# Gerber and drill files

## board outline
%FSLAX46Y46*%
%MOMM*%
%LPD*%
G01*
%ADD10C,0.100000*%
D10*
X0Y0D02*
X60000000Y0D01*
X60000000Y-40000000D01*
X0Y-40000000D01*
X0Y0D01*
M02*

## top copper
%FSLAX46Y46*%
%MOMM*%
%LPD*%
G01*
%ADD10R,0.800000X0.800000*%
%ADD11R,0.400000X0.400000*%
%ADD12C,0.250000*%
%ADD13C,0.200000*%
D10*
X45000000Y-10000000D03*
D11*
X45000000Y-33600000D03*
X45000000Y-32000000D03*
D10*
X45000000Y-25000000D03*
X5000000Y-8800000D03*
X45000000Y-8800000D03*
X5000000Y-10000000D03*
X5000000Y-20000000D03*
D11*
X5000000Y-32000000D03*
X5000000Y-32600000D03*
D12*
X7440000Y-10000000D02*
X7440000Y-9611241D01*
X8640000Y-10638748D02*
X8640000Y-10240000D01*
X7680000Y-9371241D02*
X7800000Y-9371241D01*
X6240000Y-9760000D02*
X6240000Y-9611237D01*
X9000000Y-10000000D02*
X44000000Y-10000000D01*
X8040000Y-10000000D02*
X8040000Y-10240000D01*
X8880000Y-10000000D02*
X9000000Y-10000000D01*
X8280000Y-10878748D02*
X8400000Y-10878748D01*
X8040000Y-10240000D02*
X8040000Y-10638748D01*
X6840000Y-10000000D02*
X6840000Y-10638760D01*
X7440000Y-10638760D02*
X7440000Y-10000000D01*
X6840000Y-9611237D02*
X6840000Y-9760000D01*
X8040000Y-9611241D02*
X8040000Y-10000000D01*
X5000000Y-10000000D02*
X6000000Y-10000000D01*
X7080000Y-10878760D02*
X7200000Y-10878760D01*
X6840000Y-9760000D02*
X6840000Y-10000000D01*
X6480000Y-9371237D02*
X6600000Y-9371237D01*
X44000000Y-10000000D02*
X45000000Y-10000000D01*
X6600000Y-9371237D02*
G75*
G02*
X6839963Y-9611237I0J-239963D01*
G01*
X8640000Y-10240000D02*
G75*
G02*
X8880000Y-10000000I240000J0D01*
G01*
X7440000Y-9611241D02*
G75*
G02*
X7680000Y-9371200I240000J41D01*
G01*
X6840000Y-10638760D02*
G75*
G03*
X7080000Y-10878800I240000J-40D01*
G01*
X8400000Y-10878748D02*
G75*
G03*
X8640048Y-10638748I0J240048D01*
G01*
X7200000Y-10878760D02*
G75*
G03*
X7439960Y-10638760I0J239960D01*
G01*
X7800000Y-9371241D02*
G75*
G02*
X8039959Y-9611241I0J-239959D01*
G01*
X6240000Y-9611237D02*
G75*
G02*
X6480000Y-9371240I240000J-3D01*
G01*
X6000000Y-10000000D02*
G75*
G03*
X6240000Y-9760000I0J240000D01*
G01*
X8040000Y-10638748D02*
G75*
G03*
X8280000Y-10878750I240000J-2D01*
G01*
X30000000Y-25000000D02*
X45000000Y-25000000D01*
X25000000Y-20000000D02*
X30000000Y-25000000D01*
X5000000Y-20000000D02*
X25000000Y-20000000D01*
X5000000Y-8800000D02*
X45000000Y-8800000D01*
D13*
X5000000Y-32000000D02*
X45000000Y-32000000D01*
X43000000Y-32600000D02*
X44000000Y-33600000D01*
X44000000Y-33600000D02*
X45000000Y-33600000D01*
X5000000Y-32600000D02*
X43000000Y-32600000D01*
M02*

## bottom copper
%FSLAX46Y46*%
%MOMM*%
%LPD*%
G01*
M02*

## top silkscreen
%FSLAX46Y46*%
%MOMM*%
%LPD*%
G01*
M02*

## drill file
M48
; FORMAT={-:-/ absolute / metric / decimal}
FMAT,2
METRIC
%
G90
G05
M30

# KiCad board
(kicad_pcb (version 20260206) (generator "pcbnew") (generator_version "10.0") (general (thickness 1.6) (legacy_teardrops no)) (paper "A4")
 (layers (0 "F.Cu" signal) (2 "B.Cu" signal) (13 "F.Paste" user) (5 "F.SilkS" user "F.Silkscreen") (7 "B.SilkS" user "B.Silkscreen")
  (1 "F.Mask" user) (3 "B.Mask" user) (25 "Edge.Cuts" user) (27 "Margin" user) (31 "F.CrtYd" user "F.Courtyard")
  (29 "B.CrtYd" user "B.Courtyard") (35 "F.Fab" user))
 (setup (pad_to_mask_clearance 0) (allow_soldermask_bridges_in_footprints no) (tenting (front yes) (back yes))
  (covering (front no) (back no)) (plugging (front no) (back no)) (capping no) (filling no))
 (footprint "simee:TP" (layer "F.Cu") (at 45 10)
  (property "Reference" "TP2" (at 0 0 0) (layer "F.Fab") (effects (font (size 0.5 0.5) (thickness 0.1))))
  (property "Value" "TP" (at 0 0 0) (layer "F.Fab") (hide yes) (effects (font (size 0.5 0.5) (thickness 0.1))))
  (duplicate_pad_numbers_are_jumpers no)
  (pad "1" smd rect (at 0 0) (size 0.8 0.8) (layers "F.Cu" "F.Mask") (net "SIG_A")))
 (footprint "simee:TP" (layer "F.Cu") (at 45 33.6)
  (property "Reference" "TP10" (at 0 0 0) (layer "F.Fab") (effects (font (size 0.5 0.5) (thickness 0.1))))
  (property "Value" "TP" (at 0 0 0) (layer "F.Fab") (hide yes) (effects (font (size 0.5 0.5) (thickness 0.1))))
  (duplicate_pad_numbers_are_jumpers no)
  (pad "1" smd rect (at 0 0) (size 0.4 0.4) (layers "F.Cu" "F.Mask") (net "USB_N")))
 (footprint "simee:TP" (layer "F.Cu") (at 45 32)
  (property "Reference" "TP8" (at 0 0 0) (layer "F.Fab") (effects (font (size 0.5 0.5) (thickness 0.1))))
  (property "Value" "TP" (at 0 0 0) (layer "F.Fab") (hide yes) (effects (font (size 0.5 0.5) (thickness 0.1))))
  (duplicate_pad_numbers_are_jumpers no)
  (pad "1" smd rect (at 0 0) (size 0.4 0.4) (layers "F.Cu" "F.Mask") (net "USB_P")))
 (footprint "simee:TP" (layer "F.Cu") (at 45 25)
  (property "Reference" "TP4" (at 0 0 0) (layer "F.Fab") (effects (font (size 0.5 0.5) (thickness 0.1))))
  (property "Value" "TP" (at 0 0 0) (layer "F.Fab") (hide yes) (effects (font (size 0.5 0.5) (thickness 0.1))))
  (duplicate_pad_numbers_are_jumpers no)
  (pad "1" smd rect (at 0 0) (size 0.8 0.8) (layers "F.Cu" "F.Mask") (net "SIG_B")))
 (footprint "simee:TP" (layer "F.Cu") (at 5 8.8)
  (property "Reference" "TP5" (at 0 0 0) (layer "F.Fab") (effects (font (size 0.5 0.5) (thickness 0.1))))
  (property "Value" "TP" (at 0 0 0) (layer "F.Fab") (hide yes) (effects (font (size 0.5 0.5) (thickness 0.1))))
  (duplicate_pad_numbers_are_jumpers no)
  (pad "1" smd rect (at 0 0) (size 0.8 0.8) (layers "F.Cu" "F.Mask") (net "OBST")))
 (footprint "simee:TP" (layer "F.Cu") (at 45 8.8)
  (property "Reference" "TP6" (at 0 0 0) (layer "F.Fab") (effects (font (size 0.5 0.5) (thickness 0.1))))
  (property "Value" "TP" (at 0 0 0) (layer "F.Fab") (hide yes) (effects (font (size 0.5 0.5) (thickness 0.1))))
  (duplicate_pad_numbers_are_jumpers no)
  (pad "1" smd rect (at 0 0) (size 0.8 0.8) (layers "F.Cu" "F.Mask") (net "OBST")))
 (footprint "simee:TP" (layer "F.Cu") (at 5 10)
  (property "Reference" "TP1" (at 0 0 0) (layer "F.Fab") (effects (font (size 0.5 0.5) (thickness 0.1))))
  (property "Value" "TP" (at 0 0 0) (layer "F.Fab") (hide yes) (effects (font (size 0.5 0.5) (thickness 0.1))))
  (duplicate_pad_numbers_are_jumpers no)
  (pad "1" smd rect (at 0 0) (size 0.8 0.8) (layers "F.Cu" "F.Mask") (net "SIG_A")))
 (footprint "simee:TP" (layer "F.Cu") (at 5 20)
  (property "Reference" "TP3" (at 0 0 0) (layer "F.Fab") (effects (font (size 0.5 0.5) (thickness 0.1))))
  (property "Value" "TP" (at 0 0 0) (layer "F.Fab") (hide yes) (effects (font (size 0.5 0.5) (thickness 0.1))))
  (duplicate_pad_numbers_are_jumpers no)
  (pad "1" smd rect (at 0 0) (size 0.8 0.8) (layers "F.Cu" "F.Mask") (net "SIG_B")))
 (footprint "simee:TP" (layer "F.Cu") (at 5 32)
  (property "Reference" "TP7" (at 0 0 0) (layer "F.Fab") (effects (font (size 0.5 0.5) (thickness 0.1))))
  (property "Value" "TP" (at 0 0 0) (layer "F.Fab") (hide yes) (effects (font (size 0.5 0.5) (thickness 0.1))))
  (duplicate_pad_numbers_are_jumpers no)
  (pad "1" smd rect (at 0 0) (size 0.4 0.4) (layers "F.Cu" "F.Mask") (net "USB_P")))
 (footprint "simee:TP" (layer "F.Cu") (at 5 32.6)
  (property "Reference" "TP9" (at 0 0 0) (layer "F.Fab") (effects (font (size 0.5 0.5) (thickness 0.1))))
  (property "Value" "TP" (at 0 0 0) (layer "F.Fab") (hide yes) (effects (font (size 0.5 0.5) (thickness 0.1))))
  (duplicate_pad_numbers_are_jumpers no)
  (pad "1" smd rect (at 0 0) (size 0.4 0.4) (layers "F.Cu" "F.Mask") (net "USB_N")))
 (gr_rect (start 0 0) (end 60 40) (stroke (width 0.1) (type default)) (fill no) (layer "Edge.Cuts"))
 (segment (start 7.44 10) (end 7.44 9.611241) (width 0.25) (layer "F.Cu") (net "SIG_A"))
 (segment (start 8.64 10.638748) (end 8.64 10.24) (width 0.25) (layer "F.Cu") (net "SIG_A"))
 (segment (start 7.68 9.371241) (end 7.8 9.371241) (width 0.25) (layer "F.Cu") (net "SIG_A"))
 (segment (start 6.24 9.76) (end 6.24 9.611237) (width 0.25) (layer "F.Cu") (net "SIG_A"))
 (segment (start 9 10) (end 44 10) (width 0.25) (layer "F.Cu") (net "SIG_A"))
 (segment (start 8.04 10) (end 8.04 10.24) (width 0.25) (layer "F.Cu") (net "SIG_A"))
 (segment (start 8.88 10) (end 9 10) (width 0.25) (layer "F.Cu") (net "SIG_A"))
 (segment (start 8.28 10.878748) (end 8.4 10.878748) (width 0.25) (layer "F.Cu") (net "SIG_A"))
 (segment (start 8.04 10.24) (end 8.04 10.638748) (width 0.25) (layer "F.Cu") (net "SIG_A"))
 (segment (start 6.84 10) (end 6.84 10.63876) (width 0.25) (layer "F.Cu") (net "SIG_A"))
 (segment (start 7.44 10.63876) (end 7.44 10) (width 0.25) (layer "F.Cu") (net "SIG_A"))
 (segment (start 6.84 9.611237) (end 6.84 9.76) (width 0.25) (layer "F.Cu") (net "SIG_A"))
 (segment (start 8.04 9.611241) (end 8.04 10) (width 0.25) (layer "F.Cu") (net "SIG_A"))
 (segment (start 5 10) (end 6 10) (width 0.25) (layer "F.Cu") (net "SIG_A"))
 (segment (start 7.08 10.87876) (end 7.2 10.87876) (width 0.25) (layer "F.Cu") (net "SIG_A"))
 (segment (start 6.84 9.76) (end 6.84 10) (width 0.25) (layer "F.Cu") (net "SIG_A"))
 (segment (start 6.48 9.371237) (end 6.6 9.371237) (width 0.25) (layer "F.Cu") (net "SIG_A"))
 (segment (start 44 10) (end 45 10) (width 0.25) (layer "F.Cu") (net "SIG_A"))
 (arc (start 6.6 9.371237) (mid 6.769706 9.441531) (end 6.84 9.611237) (width 0.25) (layer "F.Cu") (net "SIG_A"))
 (arc (start 8.64 10.24) (mid 8.710294 10.070294) (end 8.88 10) (width 0.25) (layer "F.Cu") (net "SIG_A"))
 (arc (start 7.44 9.611241) (mid 7.510294 9.441535) (end 7.68 9.371241) (width 0.25) (layer "F.Cu") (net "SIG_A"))
 (arc (start 6.84 10.63876) (mid 6.910294 10.808466) (end 7.08 10.87876) (width 0.25) (layer "F.Cu") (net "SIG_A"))
 (arc (start 8.4 10.878748) (mid 8.569706 10.808454) (end 8.64 10.638748) (width 0.25) (layer "F.Cu") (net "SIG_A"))
 (arc (start 7.2 10.87876) (mid 7.369706 10.808466) (end 7.44 10.63876) (width 0.25) (layer "F.Cu") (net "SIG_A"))
 (arc (start 7.8 9.371241) (mid 7.969706 9.441535) (end 8.04 9.611241) (width 0.25) (layer "F.Cu") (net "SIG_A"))
 (arc (start 6.24 9.611237) (mid 6.310294 9.441531) (end 6.48 9.371237) (width 0.25) (layer "F.Cu") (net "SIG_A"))
 (arc (start 6 10) (mid 6.169706 9.929706) (end 6.24 9.76) (width 0.25) (layer "F.Cu") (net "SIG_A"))
 (arc (start 8.04 10.638748) (mid 8.110294 10.808454) (end 8.28 10.878748) (width 0.25) (layer "F.Cu") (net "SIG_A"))
 (segment (start 30 25) (end 45 25) (width 0.25) (layer "F.Cu") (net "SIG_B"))
 (segment (start 25 20) (end 30 25) (width 0.25) (layer "F.Cu") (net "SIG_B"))
 (segment (start 5 20) (end 25 20) (width 0.25) (layer "F.Cu") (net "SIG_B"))
 (segment (start 5 8.8) (end 45 8.8) (width 0.25) (layer "F.Cu") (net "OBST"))
 (segment (start 5 32) (end 45 32) (width 0.2) (layer "F.Cu") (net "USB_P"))
 (segment (start 43 32.6) (end 44 33.6) (width 0.2) (layer "F.Cu") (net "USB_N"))
 (segment (start 44 33.6) (end 45 33.6) (width 0.2) (layer "F.Cu") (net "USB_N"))
 (segment (start 5 32.6) (end 43 32.6) (width 0.2) (layer "F.Cu") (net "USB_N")))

